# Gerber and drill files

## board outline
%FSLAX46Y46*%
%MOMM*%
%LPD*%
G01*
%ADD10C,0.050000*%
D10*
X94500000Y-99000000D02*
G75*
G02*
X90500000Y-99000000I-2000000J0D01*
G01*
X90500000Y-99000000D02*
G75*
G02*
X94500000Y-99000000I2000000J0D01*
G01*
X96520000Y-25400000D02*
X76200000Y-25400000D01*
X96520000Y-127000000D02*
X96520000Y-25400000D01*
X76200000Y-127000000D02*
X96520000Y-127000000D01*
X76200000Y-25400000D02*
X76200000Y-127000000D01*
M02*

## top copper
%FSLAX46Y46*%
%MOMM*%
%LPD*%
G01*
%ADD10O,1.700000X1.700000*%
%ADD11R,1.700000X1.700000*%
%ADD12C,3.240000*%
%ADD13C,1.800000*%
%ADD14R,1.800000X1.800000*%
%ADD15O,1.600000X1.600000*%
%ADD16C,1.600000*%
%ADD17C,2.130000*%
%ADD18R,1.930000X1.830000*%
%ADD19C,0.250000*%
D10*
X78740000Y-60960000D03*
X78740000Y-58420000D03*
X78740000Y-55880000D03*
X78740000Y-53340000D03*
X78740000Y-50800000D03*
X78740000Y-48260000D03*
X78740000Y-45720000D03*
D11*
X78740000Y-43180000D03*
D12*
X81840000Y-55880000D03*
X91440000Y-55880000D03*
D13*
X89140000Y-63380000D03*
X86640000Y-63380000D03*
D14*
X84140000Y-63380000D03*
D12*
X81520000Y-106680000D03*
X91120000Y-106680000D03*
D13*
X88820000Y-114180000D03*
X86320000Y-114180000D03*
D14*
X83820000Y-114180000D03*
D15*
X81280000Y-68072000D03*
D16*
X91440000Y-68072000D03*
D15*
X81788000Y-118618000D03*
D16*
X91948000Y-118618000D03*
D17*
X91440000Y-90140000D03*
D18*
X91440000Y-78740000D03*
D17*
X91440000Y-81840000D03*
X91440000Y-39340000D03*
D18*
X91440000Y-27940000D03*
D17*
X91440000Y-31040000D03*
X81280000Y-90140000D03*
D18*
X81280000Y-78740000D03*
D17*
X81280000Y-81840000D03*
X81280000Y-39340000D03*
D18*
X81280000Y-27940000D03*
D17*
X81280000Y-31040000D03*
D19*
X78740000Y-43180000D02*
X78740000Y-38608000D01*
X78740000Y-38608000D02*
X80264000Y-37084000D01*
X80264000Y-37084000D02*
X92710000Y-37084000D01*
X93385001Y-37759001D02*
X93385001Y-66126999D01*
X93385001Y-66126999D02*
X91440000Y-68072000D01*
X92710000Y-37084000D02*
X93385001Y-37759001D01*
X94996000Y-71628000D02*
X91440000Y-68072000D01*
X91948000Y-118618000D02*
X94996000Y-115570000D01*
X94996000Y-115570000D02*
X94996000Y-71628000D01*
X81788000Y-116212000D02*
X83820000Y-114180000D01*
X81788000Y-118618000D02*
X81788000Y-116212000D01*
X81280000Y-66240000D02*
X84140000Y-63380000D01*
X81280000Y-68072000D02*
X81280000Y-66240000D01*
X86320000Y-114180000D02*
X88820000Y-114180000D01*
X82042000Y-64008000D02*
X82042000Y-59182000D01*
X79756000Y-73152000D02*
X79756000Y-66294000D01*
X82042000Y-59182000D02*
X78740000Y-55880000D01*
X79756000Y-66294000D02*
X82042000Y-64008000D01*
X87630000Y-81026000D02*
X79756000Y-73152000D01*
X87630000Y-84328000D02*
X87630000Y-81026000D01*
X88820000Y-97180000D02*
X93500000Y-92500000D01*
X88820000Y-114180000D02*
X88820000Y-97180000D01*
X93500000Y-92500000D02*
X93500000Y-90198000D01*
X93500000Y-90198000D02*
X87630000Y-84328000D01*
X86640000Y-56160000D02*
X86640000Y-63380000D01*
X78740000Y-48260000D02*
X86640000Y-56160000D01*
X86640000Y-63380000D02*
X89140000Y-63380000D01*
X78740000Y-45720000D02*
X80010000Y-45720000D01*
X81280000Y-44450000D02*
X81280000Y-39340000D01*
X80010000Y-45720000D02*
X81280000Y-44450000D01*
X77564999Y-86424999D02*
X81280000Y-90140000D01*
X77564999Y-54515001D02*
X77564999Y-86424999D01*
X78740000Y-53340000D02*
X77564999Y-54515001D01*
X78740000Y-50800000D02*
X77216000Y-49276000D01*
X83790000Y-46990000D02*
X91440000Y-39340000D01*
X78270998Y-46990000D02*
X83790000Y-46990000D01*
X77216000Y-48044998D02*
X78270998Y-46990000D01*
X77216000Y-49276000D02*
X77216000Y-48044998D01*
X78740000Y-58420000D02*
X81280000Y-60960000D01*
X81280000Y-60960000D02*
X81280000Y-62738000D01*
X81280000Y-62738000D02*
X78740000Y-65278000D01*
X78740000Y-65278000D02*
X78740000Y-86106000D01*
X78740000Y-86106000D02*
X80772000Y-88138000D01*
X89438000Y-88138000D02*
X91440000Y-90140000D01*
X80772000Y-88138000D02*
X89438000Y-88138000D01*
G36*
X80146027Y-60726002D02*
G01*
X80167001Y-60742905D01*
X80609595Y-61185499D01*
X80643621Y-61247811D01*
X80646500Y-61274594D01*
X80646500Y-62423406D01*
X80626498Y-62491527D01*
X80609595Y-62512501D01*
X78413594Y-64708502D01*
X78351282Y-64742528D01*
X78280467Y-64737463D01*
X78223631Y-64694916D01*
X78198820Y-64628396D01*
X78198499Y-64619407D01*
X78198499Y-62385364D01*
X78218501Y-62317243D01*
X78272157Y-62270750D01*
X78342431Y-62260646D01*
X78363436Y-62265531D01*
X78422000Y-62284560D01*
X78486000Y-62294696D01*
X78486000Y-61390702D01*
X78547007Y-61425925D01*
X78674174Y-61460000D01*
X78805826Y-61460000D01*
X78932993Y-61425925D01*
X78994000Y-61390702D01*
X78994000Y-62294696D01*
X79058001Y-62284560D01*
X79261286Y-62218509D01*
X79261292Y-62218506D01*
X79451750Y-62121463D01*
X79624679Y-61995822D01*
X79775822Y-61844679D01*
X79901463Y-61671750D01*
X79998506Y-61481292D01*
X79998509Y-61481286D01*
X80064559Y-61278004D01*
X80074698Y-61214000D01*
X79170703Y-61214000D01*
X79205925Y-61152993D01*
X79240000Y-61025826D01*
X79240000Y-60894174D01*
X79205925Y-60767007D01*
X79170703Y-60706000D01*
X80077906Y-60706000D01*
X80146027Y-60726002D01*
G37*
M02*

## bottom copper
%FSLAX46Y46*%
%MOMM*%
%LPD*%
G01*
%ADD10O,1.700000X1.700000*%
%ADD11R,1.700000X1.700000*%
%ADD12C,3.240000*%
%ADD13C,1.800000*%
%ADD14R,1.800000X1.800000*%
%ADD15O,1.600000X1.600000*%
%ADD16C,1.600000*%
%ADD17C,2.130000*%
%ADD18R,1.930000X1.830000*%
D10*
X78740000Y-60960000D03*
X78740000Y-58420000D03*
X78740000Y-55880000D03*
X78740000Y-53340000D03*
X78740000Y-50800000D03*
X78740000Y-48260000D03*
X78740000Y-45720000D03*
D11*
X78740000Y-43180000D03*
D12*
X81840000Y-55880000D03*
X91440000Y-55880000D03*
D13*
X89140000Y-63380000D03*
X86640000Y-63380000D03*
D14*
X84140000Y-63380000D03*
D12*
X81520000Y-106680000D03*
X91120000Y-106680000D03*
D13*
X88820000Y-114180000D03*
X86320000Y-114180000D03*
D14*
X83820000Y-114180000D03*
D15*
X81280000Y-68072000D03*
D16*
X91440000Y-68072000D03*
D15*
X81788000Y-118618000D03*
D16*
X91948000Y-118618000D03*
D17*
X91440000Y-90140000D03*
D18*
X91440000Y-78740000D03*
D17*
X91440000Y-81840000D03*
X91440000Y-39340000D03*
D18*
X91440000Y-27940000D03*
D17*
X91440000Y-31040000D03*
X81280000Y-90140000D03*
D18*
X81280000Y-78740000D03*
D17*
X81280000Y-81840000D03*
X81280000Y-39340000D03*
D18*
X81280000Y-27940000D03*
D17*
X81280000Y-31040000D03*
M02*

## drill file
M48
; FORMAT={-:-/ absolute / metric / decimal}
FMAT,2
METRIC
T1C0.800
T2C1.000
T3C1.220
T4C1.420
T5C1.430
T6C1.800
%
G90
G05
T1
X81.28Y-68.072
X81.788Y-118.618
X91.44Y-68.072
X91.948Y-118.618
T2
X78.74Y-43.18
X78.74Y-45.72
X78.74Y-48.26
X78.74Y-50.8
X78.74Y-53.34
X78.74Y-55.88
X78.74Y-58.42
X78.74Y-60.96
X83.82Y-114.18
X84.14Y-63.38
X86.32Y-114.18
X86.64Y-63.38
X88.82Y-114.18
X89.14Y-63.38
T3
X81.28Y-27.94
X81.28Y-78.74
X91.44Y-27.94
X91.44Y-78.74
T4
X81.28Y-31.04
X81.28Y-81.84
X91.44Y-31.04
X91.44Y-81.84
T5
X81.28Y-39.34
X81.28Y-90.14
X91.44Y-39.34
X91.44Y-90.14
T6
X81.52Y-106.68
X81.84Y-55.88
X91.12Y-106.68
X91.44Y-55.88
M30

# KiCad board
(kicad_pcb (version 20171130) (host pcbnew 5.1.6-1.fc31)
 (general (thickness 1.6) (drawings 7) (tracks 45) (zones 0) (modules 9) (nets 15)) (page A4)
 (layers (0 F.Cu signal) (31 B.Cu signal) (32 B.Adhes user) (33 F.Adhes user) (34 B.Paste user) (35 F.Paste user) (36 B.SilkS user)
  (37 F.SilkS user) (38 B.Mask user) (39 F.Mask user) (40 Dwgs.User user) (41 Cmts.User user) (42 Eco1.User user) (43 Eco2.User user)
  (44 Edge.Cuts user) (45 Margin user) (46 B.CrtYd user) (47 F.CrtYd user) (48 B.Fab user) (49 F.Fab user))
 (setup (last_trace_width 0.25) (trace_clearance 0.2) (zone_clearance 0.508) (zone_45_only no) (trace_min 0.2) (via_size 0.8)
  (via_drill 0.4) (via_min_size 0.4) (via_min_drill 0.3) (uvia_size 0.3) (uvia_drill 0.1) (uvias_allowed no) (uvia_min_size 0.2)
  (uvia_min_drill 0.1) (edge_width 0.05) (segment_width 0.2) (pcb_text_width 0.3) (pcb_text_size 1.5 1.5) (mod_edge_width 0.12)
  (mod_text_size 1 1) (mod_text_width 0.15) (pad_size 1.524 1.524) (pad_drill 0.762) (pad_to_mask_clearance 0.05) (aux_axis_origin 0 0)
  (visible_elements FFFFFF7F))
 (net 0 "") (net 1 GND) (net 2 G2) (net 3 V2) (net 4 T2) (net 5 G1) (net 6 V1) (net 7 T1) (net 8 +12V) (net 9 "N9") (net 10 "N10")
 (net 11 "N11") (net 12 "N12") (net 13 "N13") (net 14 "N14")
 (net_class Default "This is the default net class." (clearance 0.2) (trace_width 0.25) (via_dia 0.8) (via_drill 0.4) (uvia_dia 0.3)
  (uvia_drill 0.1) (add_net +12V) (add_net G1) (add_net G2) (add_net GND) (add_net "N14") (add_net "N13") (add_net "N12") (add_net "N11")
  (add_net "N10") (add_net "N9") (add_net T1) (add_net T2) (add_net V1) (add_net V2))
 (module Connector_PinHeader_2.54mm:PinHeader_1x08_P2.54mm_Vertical (layer F.Cu) (at 78.74 43.18)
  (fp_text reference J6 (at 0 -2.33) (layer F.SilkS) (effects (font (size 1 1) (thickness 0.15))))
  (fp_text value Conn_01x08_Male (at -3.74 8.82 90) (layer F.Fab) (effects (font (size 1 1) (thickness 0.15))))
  (pad 8 thru_hole oval (at 0 17.78) (size 1.7 1.7) (drill 1) (layers *.Cu *.Mask) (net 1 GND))
  (pad 7 thru_hole oval (at 0 15.24) (size 1.7 1.7) (drill 1) (layers *.Cu *.Mask) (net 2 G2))
  (pad 6 thru_hole oval (at 0 12.7) (size 1.7 1.7) (drill 1) (layers *.Cu *.Mask) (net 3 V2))
  (pad 5 thru_hole oval (at 0 10.16) (size 1.7 1.7) (drill 1) (layers *.Cu *.Mask) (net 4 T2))
  (pad 4 thru_hole oval (at 0 7.62) (size 1.7 1.7) (drill 1) (layers *.Cu *.Mask) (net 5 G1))
  (pad 3 thru_hole oval (at 0 5.08) (size 1.7 1.7) (drill 1) (layers *.Cu *.Mask) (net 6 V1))
  (pad 2 thru_hole oval (at 0 2.54) (size 1.7 1.7) (drill 1) (layers *.Cu *.Mask) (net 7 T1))
  (pad 1 thru_hole rect (at 0 0) (size 1.7 1.7) (drill 1) (layers *.Cu *.Mask) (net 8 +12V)))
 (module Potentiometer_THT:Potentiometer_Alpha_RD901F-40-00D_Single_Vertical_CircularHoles (layer F.Cu) (at 84.14 63.38 90)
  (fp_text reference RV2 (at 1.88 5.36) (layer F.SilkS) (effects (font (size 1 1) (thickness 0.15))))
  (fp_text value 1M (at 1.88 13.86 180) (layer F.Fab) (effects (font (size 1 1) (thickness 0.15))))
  (pad "" thru_hole circle (at 7.5 -2.3 180) (size 3.24 3.24) (drill 1.8) (layers *.Cu *.Mask))
  (pad "" thru_hole circle (at 7.5 7.3 180) (size 3.24 3.24) (drill 1.8) (layers *.Cu *.Mask))
  (pad 3 thru_hole circle (at 0 5 180) (size 1.8 1.8) (drill 1) (layers *.Cu *.Mask) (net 6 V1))
  (pad 2 thru_hole circle (at 0 2.5 180) (size 1.8 1.8) (drill 1) (layers *.Cu *.Mask) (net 6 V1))
  (pad 1 thru_hole rect (at 0 0 180) (size 1.8 1.8) (drill 1) (layers *.Cu *.Mask) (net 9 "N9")))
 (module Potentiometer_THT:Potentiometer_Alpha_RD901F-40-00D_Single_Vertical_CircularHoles (layer F.Cu) (at 83.82 114.18 90)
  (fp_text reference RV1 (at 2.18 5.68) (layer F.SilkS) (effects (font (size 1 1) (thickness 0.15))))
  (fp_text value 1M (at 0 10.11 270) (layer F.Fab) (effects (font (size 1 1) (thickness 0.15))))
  (pad "" thru_hole circle (at 7.5 -2.3 180) (size 3.24 3.24) (drill 1.8) (layers *.Cu *.Mask))
  (pad "" thru_hole circle (at 7.5 7.3 180) (size 3.24 3.24) (drill 1.8) (layers *.Cu *.Mask))
  (pad 3 thru_hole circle (at 0 5 180) (size 1.8 1.8) (drill 1) (layers *.Cu *.Mask) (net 3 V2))
  (pad 2 thru_hole circle (at 0 2.5 180) (size 1.8 1.8) (drill 1) (layers *.Cu *.Mask) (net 3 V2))
  (pad 1 thru_hole rect (at 0 0 180) (size 1.8 1.8) (drill 1) (layers *.Cu *.Mask) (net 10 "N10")))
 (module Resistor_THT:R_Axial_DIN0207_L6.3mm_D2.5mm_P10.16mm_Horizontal (layer F.Cu) (at 91.44 68.072 180)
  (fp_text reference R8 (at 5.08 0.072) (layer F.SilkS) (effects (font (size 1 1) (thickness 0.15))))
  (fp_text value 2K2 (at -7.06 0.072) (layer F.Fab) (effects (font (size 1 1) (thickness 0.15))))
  (pad 2 thru_hole oval (at 10.16 0 180) (size 1.6 1.6) (drill 0.8) (layers *.Cu *.Mask) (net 9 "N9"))
  (pad 1 thru_hole circle (at 0 0 180) (size 1.6 1.6) (drill 0.8) (layers *.Cu *.Mask) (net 8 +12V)))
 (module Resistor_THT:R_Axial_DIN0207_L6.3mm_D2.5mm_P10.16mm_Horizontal (layer F.Cu) (at 91.948 118.618 180)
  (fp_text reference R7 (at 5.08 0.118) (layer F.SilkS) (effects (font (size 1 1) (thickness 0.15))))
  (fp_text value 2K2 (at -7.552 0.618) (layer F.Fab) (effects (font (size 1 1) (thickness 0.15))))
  (pad 2 thru_hole oval (at 10.16 0 180) (size 1.6 1.6) (drill 0.8) (layers *.Cu *.Mask) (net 10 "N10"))
  (pad 1 thru_hole circle (at 0 0 180) (size 1.6 1.6) (drill 0.8) (layers *.Cu *.Mask) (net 8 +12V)))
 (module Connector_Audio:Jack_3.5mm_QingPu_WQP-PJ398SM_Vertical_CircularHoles (layer F.Cu) (at 91.44 78.74)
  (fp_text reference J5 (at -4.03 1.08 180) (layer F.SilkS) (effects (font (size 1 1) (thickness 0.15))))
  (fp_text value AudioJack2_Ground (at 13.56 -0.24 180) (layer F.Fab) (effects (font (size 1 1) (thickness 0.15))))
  (pad T thru_hole circle (at 0 11.4 180) (size 2.13 2.13) (drill 1.43) (layers *.Cu *.Mask) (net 2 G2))
  (pad S thru_hole rect (at 0 0 180) (size 1.93 1.83) (drill 1.22) (layers *.Cu *.Mask) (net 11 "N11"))
  (pad TN thru_hole circle (at 0 3.1 180) (size 2.13 2.13) (drill 1.42) (layers *.Cu *.Mask)))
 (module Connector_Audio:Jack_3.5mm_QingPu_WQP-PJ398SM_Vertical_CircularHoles (layer F.Cu) (at 91.44 27.94)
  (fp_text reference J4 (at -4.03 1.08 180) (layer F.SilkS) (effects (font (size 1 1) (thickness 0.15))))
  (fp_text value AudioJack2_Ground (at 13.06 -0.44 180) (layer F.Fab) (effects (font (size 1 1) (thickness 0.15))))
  (pad T thru_hole circle (at 0 11.4 180) (size 2.13 2.13) (drill 1.43) (layers *.Cu *.Mask) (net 5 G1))
  (pad S thru_hole rect (at 0 0 180) (size 1.93 1.83) (drill 1.22) (layers *.Cu *.Mask) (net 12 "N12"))
  (pad TN thru_hole circle (at 0 3.1 180) (size 2.13 2.13) (drill 1.42) (layers *.Cu *.Mask)))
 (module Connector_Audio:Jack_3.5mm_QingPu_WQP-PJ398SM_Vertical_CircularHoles (layer F.Cu) (at 81.28 78.74)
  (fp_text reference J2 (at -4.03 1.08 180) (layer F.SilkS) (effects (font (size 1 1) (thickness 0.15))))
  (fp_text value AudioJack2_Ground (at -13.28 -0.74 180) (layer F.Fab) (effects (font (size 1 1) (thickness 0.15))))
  (pad T thru_hole circle (at 0 11.4 180) (size 2.13 2.13) (drill 1.43) (layers *.Cu *.Mask) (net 4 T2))
  (pad S thru_hole rect (at 0 0 180) (size 1.93 1.83) (drill 1.22) (layers *.Cu *.Mask) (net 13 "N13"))
  (pad TN thru_hole circle (at 0 3.1 180) (size 2.13 2.13) (drill 1.42) (layers *.Cu *.Mask)))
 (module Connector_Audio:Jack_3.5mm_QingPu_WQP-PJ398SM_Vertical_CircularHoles (layer F.Cu) (at 81.28 27.94)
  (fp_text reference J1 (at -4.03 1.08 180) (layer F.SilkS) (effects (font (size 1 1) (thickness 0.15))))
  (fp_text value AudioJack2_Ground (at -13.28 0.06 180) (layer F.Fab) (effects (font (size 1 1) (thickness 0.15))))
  (pad T thru_hole circle (at 0 11.4 180) (size 2.13 2.13) (drill 1.43) (layers *.Cu *.Mask) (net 7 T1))
  (pad S thru_hole rect (at 0 0 180) (size 1.93 1.83) (drill 1.22) (layers *.Cu *.Mask) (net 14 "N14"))
  (pad TN thru_hole circle (at 0 3.1 180) (size 2.13 2.13) (drill 1.42) (layers *.Cu *.Mask)))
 (gr_circle (center 92.5 99) (end 94.5 99) (layer Edge.Cuts) (width 0.05))
 (gr_line (start 96.52 25.4) (end 76.2 25.4) (layer Edge.Cuts) (width 0.05))
 (gr_line (start 96.52 127) (end 96.52 25.4) (layer Edge.Cuts) (width 0.05))
 (gr_line (start 76.2 127) (end 96.52 127) (layer Edge.Cuts) (width 0.05))
 (gr_line (start 76.2 25.4) (end 76.2 127) (layer Edge.Cuts) (width 0.05))
 (segment (start 78.74 43.18) (end 78.74 38.608) (width 0.25) (layer F.Cu) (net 8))
 (segment (start 78.74 38.608) (end 80.264 37.084) (width 0.25) (layer F.Cu) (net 8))
 (segment (start 80.264 37.084) (end 92.71 37.084) (width 0.25) (layer F.Cu) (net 8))
 (segment (start 93.385001 37.759001) (end 93.385001 66.126999) (width 0.25) (layer F.Cu) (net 8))
 (segment (start 93.385001 66.126999) (end 91.44 68.072) (width 0.25) (layer F.Cu) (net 8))
 (segment (start 92.71 37.084) (end 93.385001 37.759001) (width 0.25) (layer F.Cu) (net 8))
 (segment (start 94.996 71.628) (end 91.44 68.072) (width 0.25) (layer F.Cu) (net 8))
 (segment (start 91.948 118.618) (end 94.996 115.57) (width 0.25) (layer F.Cu) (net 8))
 (segment (start 94.996 115.57) (end 94.996 71.628) (width 0.25) (layer F.Cu) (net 8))
 (segment (start 81.788 116.212) (end 83.82 114.18) (width 0.25) (layer F.Cu) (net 10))
 (segment (start 81.788 118.618) (end 81.788 116.212) (width 0.25) (layer F.Cu) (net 10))
 (segment (start 81.28 66.24) (end 84.14 63.38) (width 0.25) (layer F.Cu) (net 9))
 (segment (start 81.28 68.072) (end 81.28 66.24) (width 0.25) (layer F.Cu) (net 9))
 (segment (start 86.32 114.18) (end 88.82 114.18) (width 0.25) (layer F.Cu) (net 3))
 (segment (start 82.042 64.008) (end 82.042 59.182) (width 0.25) (layer F.Cu) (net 3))
 (segment (start 79.756 73.152) (end 79.756 66.294) (width 0.25) (layer F.Cu) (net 3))
 (segment (start 82.042 59.182) (end 78.74 55.88) (width 0.25) (layer F.Cu) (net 3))
 (segment (start 79.756 66.294) (end 82.042 64.008) (width 0.25) (layer F.Cu) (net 3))
 (segment (start 87.63 81.026) (end 79.756 73.152) (width 0.25) (layer F.Cu) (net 3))
 (segment (start 87.63 84.328) (end 87.63 81.026) (width 0.25) (layer F.Cu) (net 3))
 (segment (start 88.82 97.18) (end 93.5 92.5) (width 0.25) (layer F.Cu) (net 3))
 (segment (start 88.82 114.18) (end 88.82 97.18) (width 0.25) (layer F.Cu) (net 3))
 (segment (start 93.5 92.5) (end 93.5 90.198) (width 0.25) (layer F.Cu) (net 3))
 (segment (start 93.5 90.198) (end 87.63 84.328) (width 0.25) (layer F.Cu) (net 3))
 (segment (start 86.64 56.16) (end 86.64 63.38) (width 0.25) (layer F.Cu) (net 6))
 (segment (start 78.74 48.26) (end 86.64 56.16) (width 0.25) (layer F.Cu) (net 6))
 (segment (start 86.64 63.38) (end 89.14 63.38) (width 0.25) (layer F.Cu) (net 6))
 (segment (start 78.74 45.72) (end 80.01 45.72) (width 0.25) (layer F.Cu) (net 7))
 (segment (start 81.28 44.45) (end 81.28 39.34) (width 0.25) (layer F.Cu) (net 7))
 (segment (start 80.01 45.72) (end 81.28 44.45) (width 0.25) (layer F.Cu) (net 7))
 (segment (start 77.564999 86.424999) (end 81.28 90.14) (width 0.25) (layer F.Cu) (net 4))
 (segment (start 77.564999 54.515001) (end 77.564999 86.424999) (width 0.25) (layer F.Cu) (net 4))
 (segment (start 78.74 53.34) (end 77.564999 54.515001) (width 0.25) (layer F.Cu) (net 4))
 (segment (start 78.74 50.8) (end 77.216 49.276) (width 0.25) (layer F.Cu) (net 5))
 (segment (start 83.79 46.99) (end 91.44 39.34) (width 0.25) (layer F.Cu) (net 5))
 (segment (start 78.270998 46.99) (end 83.79 46.99) (width 0.25) (layer F.Cu) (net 5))
 (segment (start 77.216 48.044998) (end 78.270998 46.99) (width 0.25) (layer F.Cu) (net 5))
 (segment (start 77.216 49.276) (end 77.216 48.044998) (width 0.25) (layer F.Cu) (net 5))
 (segment (start 78.74 58.42) (end 81.28 60.96) (width 0.25) (layer F.Cu) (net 2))
 (segment (start 81.28 60.96) (end 81.28 62.738) (width 0.25) (layer F.Cu) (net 2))
 (segment (start 81.28 62.738) (end 78.74 65.278) (width 0.25) (layer F.Cu) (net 2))
 (segment (start 78.74 65.278) (end 78.74 86.106) (width 0.25) (layer F.Cu) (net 2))
 (segment (start 78.74 86.106) (end 80.772 88.138) (width 0.25) (layer F.Cu) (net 2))
 (segment (start 89.438 88.138) (end 91.44 90.14) (width 0.25) (layer F.Cu) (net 2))
 (segment (start 80.772 88.138) (end 89.438 88.138) (width 0.25) (layer F.Cu) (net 2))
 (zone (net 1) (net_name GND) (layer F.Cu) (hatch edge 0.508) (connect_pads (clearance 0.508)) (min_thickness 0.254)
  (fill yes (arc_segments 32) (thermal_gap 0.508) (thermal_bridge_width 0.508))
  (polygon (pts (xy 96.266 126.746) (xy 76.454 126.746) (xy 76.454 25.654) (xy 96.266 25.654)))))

